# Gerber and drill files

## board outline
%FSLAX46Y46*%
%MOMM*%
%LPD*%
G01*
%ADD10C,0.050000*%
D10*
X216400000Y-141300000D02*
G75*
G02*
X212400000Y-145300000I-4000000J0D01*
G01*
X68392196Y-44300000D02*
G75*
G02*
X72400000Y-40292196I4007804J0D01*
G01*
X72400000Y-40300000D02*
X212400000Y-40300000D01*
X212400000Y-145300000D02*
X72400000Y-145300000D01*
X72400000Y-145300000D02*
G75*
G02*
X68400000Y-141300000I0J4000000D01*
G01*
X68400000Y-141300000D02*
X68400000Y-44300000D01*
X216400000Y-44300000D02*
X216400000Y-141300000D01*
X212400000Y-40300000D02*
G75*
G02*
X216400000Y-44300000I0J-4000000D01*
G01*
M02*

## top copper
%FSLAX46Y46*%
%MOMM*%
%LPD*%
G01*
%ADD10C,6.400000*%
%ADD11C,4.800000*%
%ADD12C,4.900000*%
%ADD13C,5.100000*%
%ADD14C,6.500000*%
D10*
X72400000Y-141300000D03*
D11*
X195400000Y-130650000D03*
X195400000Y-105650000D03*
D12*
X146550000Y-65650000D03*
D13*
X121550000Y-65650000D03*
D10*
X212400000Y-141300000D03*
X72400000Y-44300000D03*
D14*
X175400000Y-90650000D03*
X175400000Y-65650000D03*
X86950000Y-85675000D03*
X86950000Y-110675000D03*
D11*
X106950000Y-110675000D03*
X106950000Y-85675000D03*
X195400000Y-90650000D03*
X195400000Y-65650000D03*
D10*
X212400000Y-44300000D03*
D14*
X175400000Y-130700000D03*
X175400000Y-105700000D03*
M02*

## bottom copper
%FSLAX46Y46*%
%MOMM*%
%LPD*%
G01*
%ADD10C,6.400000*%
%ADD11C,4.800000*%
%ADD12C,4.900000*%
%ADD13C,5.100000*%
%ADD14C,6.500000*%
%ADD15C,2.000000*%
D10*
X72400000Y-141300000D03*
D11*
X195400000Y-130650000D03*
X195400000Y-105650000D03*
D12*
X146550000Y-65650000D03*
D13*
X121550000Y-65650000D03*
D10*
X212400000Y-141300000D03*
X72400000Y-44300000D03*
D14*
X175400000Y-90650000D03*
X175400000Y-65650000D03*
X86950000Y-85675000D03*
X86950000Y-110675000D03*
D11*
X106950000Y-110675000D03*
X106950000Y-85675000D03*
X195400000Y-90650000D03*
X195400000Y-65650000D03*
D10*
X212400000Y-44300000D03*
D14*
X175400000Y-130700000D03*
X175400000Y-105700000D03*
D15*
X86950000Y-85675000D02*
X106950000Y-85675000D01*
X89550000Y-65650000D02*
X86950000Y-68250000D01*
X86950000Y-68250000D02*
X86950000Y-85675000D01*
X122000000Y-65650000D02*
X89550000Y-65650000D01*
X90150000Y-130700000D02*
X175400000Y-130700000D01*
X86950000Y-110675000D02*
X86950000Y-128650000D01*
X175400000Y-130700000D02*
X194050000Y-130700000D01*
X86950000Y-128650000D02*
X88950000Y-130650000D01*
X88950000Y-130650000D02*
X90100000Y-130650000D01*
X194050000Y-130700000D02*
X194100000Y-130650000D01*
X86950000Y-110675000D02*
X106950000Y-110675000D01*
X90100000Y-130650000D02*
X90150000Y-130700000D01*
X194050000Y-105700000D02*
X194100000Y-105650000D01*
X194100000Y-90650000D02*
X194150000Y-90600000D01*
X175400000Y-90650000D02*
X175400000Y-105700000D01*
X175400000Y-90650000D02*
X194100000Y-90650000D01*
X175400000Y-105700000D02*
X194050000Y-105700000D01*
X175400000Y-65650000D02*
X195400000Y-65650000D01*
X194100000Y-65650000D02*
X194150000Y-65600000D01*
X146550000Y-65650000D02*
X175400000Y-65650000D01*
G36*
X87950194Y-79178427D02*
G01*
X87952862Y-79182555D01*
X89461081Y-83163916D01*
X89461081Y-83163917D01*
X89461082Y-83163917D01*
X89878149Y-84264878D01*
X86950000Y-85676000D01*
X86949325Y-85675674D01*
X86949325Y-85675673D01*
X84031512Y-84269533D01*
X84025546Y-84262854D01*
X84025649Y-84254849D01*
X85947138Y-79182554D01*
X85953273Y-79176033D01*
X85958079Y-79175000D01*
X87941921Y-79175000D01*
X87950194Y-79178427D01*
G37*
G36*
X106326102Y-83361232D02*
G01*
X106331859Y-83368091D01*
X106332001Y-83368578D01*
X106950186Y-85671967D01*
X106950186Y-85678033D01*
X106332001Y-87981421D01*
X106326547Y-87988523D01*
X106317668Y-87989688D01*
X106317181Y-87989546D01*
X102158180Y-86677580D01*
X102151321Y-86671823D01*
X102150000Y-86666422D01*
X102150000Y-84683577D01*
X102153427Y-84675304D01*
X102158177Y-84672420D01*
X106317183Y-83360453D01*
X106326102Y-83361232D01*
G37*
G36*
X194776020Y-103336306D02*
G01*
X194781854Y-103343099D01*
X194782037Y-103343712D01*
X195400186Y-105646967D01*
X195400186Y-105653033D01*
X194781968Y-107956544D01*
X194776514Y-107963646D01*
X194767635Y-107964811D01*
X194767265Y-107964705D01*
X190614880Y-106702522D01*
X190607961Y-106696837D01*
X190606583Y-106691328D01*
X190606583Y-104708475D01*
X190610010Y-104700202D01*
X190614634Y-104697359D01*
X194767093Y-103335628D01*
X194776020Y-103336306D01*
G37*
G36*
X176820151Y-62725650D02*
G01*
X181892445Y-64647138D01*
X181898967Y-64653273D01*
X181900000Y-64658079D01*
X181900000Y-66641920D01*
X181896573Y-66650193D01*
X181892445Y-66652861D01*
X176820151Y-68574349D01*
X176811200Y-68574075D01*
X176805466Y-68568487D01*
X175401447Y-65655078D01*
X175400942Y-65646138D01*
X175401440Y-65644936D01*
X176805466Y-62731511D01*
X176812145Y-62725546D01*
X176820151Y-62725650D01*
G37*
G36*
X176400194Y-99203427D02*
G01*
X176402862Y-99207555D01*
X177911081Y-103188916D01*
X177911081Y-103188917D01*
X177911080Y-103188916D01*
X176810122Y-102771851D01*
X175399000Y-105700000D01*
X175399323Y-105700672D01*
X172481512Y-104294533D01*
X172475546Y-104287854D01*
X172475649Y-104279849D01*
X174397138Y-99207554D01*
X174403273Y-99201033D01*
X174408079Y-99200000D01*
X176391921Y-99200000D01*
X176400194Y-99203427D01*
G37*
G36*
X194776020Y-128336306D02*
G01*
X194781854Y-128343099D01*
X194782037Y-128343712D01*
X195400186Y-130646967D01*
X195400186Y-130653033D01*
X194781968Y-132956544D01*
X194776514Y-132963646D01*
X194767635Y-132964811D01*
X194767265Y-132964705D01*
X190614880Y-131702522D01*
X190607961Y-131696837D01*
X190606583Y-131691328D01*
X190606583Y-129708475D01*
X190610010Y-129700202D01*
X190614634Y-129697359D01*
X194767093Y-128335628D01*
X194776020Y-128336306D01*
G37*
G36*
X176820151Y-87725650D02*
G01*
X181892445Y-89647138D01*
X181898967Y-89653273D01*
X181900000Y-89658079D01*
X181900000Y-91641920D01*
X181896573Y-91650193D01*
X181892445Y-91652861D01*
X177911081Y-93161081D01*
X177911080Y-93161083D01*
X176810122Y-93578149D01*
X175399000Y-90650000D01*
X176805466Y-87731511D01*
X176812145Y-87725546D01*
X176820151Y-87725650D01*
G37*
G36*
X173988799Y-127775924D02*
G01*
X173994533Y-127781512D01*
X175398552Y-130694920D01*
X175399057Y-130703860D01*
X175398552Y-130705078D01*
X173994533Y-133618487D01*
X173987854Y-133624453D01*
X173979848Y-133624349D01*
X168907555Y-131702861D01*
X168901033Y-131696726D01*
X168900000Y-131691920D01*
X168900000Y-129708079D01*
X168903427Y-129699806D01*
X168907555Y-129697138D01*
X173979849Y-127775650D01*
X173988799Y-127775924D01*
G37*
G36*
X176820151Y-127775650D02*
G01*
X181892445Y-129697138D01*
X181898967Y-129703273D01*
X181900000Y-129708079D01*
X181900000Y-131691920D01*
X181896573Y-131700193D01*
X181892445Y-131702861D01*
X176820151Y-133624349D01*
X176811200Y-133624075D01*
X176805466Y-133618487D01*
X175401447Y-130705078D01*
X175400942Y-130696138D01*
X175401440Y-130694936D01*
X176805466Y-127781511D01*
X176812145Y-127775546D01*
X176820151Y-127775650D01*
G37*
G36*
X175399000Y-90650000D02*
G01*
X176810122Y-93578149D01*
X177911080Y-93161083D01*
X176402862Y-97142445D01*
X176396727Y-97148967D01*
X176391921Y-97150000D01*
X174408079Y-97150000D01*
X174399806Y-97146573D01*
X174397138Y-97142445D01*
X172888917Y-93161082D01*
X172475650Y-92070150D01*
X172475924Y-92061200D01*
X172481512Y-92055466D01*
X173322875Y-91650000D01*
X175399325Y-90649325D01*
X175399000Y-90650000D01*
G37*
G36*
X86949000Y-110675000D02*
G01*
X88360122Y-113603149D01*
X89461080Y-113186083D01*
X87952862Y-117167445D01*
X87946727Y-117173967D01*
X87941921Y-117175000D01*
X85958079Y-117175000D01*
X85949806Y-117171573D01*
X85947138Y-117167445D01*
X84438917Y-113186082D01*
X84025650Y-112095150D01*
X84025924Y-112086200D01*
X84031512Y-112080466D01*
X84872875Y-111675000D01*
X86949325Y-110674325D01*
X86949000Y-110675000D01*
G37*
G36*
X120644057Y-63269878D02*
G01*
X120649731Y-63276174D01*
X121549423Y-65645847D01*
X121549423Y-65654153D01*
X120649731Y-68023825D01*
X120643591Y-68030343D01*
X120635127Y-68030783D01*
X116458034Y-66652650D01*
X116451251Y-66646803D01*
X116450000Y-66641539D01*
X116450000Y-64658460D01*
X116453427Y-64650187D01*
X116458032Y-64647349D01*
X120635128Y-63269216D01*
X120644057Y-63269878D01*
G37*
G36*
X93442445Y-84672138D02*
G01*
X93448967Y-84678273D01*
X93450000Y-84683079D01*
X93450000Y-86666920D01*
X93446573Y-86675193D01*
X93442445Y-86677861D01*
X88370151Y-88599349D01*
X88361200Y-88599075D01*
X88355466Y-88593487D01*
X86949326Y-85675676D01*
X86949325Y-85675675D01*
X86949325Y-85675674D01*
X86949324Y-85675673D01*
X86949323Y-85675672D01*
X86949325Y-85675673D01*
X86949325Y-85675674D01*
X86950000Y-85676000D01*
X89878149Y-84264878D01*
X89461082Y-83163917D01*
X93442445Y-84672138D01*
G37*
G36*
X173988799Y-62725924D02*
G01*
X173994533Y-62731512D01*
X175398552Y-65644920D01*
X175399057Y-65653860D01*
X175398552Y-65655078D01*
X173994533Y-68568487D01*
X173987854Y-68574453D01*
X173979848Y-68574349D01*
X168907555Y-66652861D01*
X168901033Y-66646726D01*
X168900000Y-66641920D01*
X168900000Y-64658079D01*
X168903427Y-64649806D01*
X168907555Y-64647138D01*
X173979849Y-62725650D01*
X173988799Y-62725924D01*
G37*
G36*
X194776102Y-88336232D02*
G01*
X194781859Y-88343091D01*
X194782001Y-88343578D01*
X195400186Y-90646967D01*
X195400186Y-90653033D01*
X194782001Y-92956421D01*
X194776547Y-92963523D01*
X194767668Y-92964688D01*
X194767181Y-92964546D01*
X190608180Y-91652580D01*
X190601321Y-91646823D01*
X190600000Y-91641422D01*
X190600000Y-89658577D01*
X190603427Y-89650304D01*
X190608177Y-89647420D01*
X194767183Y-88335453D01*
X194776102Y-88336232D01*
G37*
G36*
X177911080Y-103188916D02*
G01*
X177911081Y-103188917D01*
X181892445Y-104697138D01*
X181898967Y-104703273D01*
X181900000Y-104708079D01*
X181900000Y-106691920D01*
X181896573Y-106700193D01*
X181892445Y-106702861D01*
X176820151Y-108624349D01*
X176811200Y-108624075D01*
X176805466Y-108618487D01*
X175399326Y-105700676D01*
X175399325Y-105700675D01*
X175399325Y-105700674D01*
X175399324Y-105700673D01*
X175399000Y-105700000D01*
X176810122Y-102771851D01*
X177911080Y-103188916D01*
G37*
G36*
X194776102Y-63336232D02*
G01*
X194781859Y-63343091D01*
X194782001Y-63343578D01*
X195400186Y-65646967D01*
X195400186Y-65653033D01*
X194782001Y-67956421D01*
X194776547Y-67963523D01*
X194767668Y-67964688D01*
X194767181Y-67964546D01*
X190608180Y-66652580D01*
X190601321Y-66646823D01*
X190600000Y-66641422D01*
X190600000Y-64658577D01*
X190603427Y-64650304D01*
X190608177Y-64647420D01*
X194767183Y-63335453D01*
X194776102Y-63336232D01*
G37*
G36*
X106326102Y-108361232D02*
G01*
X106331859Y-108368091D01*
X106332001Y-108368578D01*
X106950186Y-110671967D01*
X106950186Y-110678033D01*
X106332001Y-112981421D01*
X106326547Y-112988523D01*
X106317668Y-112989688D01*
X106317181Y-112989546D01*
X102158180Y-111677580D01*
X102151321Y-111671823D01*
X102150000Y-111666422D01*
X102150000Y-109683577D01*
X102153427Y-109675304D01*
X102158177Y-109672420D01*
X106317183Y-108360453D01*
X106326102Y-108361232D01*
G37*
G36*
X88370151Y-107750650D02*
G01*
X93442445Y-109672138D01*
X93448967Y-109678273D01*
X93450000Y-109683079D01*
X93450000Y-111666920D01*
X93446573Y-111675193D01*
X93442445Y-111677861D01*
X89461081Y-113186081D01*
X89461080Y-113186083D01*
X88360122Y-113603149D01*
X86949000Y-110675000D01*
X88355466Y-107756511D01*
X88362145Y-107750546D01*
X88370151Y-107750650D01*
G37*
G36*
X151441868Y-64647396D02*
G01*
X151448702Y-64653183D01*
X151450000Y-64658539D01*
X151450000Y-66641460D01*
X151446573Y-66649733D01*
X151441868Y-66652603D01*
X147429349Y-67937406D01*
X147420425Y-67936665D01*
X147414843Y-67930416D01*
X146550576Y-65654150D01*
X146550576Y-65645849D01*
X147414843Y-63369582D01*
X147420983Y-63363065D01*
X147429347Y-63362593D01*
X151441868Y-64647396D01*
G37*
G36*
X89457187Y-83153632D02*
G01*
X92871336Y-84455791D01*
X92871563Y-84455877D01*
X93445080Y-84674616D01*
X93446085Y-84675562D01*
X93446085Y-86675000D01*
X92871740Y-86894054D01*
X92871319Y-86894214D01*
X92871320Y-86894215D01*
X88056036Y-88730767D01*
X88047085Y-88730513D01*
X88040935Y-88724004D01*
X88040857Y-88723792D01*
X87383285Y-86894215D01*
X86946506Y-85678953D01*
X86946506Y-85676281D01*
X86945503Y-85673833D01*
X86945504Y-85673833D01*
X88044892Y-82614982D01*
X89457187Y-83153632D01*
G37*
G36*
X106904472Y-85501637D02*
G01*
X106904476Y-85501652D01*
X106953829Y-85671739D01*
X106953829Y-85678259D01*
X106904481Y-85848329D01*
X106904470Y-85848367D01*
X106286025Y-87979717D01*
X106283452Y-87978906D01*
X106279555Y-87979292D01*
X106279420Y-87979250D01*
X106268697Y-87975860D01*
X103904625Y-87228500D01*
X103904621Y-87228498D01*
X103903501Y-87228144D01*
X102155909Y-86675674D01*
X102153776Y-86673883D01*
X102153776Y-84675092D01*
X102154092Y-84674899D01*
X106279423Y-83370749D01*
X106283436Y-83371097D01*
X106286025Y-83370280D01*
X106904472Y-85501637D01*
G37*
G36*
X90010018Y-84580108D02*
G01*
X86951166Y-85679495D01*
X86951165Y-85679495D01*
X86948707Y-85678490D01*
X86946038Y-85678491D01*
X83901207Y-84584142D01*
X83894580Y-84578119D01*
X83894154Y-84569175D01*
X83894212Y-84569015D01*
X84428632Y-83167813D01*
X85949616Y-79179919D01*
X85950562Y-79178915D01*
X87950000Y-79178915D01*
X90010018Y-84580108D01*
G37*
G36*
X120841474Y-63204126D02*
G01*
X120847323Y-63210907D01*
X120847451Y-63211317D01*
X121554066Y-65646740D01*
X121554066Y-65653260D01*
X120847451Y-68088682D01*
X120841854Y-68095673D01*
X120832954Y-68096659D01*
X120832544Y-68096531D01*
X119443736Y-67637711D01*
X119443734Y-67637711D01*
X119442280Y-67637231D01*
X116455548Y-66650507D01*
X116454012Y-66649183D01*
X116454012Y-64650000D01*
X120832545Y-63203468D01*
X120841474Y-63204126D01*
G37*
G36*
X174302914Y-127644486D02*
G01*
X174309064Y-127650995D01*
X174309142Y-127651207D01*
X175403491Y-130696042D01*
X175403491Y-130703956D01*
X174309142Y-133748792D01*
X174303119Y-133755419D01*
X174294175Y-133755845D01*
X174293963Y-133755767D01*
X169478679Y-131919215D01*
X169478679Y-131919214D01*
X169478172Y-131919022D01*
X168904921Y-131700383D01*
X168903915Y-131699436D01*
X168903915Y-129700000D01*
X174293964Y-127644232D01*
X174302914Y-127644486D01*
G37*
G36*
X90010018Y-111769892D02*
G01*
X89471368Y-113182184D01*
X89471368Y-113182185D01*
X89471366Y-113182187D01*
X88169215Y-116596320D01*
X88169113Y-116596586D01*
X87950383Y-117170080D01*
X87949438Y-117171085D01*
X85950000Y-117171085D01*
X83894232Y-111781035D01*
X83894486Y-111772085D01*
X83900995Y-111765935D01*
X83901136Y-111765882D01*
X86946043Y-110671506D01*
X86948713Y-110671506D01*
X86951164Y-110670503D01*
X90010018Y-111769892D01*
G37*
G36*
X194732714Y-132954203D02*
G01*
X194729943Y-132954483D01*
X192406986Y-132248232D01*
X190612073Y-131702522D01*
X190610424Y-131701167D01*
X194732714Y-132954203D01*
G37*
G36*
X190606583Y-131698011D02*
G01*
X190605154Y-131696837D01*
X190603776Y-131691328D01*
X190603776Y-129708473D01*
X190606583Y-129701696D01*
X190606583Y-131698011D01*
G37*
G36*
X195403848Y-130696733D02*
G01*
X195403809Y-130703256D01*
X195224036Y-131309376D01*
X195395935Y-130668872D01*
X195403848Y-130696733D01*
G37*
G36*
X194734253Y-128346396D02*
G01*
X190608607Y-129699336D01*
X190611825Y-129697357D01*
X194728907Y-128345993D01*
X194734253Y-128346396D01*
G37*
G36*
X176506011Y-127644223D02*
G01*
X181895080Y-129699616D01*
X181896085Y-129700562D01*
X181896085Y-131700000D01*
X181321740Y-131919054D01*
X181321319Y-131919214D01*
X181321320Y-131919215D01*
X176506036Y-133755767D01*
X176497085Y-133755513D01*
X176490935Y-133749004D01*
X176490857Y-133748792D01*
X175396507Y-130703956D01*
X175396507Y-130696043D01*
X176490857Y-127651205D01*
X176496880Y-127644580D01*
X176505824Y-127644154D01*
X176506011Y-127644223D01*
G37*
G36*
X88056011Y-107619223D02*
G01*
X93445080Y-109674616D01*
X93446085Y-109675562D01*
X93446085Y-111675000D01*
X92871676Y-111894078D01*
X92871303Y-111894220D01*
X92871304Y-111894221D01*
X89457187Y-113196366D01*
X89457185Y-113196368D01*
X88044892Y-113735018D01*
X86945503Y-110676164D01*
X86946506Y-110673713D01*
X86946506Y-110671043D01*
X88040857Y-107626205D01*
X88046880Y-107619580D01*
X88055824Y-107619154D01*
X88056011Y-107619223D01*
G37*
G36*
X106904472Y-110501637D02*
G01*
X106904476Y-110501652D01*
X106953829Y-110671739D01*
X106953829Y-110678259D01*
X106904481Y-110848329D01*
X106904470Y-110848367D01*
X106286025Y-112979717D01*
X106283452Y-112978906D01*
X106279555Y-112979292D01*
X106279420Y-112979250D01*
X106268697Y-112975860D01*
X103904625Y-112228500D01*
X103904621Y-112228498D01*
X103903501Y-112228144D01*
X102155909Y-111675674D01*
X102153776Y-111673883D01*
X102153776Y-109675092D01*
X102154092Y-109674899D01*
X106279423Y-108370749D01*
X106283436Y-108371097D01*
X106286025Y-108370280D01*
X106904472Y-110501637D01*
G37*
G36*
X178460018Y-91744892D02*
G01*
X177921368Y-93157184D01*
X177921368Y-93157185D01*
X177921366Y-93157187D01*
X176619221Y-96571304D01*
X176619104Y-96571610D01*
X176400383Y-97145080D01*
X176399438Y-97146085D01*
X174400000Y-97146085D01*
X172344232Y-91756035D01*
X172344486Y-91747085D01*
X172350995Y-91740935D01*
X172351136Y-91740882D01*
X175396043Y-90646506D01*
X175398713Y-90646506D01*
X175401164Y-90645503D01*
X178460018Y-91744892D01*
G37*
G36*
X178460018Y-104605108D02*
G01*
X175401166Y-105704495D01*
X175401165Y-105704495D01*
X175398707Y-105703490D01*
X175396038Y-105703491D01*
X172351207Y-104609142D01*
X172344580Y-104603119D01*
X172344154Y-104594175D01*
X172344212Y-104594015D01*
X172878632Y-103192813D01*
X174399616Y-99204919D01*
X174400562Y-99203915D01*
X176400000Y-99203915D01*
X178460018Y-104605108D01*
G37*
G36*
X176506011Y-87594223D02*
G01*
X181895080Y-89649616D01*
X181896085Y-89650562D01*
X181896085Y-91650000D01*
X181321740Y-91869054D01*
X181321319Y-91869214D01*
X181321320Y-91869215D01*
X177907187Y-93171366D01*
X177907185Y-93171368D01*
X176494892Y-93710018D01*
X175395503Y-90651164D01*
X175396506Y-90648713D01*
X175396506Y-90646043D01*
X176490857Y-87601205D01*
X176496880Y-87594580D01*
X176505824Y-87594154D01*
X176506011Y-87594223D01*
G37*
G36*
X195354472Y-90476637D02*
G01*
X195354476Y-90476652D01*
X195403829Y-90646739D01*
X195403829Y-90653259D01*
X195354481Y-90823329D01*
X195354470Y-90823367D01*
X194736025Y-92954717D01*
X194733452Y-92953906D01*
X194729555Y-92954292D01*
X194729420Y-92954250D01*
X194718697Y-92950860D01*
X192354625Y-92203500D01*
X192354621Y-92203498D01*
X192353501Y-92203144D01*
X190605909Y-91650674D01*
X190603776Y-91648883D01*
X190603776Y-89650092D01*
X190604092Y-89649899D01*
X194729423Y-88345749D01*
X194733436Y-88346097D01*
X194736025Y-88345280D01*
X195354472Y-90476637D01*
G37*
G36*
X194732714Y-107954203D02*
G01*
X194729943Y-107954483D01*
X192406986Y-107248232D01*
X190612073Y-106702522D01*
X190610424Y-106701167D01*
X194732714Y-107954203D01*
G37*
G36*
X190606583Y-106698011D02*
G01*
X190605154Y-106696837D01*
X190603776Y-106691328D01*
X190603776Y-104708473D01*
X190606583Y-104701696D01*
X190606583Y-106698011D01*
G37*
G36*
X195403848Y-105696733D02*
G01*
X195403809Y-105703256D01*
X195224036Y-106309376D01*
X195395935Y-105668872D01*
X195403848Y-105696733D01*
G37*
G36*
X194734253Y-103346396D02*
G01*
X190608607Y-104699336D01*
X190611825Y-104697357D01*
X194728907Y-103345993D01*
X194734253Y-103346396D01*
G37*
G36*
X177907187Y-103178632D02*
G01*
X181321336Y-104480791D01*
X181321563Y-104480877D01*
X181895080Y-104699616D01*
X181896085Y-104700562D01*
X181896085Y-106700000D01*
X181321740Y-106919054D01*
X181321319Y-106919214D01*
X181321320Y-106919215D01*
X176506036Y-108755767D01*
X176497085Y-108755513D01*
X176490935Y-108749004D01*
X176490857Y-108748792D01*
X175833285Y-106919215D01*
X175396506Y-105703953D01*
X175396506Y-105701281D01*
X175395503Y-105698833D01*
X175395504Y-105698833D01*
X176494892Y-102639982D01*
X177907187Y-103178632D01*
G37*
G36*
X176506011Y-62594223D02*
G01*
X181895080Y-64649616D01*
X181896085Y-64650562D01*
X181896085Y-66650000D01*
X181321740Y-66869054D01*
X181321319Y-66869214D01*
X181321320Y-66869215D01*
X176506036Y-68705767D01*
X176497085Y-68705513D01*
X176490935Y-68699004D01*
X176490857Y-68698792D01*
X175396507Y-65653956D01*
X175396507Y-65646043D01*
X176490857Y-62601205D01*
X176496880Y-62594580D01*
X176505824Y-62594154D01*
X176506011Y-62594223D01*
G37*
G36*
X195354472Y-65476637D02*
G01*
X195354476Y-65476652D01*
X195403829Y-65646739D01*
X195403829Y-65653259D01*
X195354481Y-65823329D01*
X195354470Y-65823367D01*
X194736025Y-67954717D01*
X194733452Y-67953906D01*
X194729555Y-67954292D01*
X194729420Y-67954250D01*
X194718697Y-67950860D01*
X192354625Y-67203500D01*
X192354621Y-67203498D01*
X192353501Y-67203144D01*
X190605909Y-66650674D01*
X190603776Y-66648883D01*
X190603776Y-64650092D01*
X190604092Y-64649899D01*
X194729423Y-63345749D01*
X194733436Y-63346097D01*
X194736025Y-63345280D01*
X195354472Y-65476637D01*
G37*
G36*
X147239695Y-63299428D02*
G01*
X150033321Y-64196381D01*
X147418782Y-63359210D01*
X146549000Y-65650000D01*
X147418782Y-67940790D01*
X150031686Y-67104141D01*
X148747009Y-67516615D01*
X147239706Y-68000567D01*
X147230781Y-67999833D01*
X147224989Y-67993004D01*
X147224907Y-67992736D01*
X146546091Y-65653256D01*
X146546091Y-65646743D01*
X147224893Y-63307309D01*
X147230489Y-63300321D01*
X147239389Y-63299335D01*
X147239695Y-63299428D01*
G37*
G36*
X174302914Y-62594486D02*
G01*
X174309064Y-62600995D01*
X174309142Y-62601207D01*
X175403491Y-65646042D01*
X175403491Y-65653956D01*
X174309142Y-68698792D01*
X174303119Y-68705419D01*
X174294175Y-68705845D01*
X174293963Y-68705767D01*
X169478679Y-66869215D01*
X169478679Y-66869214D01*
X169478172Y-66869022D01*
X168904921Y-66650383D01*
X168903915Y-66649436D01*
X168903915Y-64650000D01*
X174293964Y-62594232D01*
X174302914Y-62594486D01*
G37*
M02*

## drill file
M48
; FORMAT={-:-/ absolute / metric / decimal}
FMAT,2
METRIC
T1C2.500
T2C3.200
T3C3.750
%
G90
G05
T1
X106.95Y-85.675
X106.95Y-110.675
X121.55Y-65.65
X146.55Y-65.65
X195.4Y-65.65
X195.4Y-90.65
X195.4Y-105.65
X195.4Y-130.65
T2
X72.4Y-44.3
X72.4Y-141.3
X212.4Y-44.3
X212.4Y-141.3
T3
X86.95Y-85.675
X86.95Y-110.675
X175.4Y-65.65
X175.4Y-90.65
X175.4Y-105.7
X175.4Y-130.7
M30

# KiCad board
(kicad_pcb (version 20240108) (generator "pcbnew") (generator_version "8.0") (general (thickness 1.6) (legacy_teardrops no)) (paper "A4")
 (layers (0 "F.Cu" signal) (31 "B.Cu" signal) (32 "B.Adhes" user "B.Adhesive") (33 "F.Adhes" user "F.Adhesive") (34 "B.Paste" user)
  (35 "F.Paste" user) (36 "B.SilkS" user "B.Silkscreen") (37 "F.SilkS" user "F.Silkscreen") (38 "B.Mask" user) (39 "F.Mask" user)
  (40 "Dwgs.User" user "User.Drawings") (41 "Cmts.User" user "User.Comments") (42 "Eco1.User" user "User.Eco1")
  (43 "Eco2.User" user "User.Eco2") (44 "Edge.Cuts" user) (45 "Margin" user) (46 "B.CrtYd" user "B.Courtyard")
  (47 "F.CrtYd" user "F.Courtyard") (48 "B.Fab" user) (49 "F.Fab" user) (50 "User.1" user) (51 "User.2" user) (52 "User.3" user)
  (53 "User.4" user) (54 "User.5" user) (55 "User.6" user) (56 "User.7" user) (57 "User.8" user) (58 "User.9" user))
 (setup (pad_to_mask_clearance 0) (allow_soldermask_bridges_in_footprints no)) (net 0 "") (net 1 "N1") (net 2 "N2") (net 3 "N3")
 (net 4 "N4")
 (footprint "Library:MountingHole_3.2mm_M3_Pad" (layer "F.Cu") (at 72.4 141.3)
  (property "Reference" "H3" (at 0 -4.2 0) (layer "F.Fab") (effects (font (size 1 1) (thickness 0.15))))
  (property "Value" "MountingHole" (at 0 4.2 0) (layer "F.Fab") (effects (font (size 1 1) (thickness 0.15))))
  (pad "1" thru_hole circle (at 0 0) (size 6.4 6.4) (drill 3.2) (layers "*.Cu" "*.Mask") (remove_unused_layers no)))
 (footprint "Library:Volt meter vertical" (layer "F.Cu") (at 195.4 118.15)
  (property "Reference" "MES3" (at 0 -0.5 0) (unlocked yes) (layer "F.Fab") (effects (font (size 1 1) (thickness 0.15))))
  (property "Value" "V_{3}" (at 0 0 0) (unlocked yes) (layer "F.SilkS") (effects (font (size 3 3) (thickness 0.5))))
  (pad "1" thru_hole circle (at 0 12.5 180) (size 4.8 4.8) (drill 2.5) (layers "*.Cu" "*.Mask") (remove_unused_layers no) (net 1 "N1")
   (teardrops (best_length_ratio 0.5) (max_length 8) (best_width_ratio 1) (max_width 8) (curve_points 0) (filter_ratio 0.9) (enabled yes)
    (allow_two_segments yes) (prefer_zone_connections yes)))
  (pad "2" thru_hole circle (at 0 -12.5 180) (size 4.8 4.8) (drill 2.5) (layers "*.Cu" "*.Mask") (remove_unused_layers no) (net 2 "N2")
   (teardrops (best_length_ratio 0.5) (max_length 8) (best_width_ratio 1) (max_width 8) (curve_points 0) (filter_ratio 0.9) (enabled yes)
    (allow_two_segments yes) (prefer_zone_connections yes))))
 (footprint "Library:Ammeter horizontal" (layer "F.Cu") (at 134.05 65.65)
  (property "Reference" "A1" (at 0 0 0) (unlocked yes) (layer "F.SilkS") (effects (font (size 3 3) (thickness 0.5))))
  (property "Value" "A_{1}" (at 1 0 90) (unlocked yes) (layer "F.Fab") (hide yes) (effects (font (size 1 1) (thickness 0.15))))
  (pad "1" thru_hole circle (at 12.5 0 270) (size 4.9 4.9) (drill 2.5) (layers "*.Cu" "*.Mask") (remove_unused_layers no) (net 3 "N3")
   (teardrops (best_length_ratio 0.5) (max_length 8) (best_width_ratio 1) (max_width 8) (curve_points 0) (filter_ratio 0.9) (enabled yes)
    (allow_two_segments yes) (prefer_zone_connections yes)))
  (pad "2" thru_hole circle (at -12.5 0 270) (size 5.1 5.1) (drill 2.5) (layers "*.Cu" "*.Mask") (remove_unused_layers no) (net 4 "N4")
   (teardrops (best_length_ratio 0.5) (max_length 8) (best_width_ratio 1) (max_width 8) (curve_points 0) (filter_ratio 0.9) (enabled yes)
    (allow_two_segments yes) (prefer_zone_connections yes))))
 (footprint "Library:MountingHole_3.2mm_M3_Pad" (layer "F.Cu") (at 212.4 141.3)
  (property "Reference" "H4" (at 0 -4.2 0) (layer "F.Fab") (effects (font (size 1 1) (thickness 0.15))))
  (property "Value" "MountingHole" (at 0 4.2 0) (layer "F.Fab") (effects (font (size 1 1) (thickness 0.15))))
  (pad "1" thru_hole circle (at 0 0) (size 6.4 6.4) (drill 3.2) (layers "*.Cu" "*.Mask") (remove_unused_layers no)))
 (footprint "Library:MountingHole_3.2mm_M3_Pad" (layer "F.Cu") (at 72.4 44.3)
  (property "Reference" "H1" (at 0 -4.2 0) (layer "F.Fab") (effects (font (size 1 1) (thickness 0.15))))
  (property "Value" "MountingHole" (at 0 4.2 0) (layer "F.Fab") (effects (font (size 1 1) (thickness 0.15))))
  (pad "1" thru_hole circle (at 0 0) (size 6.4 6.4) (drill 3.2) (layers "*.Cu" "*.Mask") (remove_unused_layers no)))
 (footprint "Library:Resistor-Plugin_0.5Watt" (layer "F.Cu") (at 175.4 78.15 180)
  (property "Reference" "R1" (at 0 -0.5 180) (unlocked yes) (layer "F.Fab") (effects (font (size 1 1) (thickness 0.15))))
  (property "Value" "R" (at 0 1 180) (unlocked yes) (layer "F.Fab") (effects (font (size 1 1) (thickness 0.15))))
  (pad "1" thru_hole circle (at 0 -12.5 180) (size 6.5 6.5) (drill 3.75) (layers "*.Cu" "*.Mask") (remove_unused_layers no) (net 2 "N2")
   (teardrops (best_length_ratio 0.5) (max_length 8) (best_width_ratio 1) (max_width 8) (curve_points 0) (filter_ratio 0.9) (enabled yes)
    (allow_two_segments yes) (prefer_zone_connections yes)))
  (pad "2" thru_hole circle (at 0 12.5 180) (size 6.5 6.5) (drill 3.75) (layers "*.Cu" "*.Mask") (remove_unused_layers no) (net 3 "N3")
   (teardrops (best_length_ratio 0.5) (max_length 8) (best_width_ratio 1) (max_width 8) (curve_points 0) (filter_ratio 0.9) (enabled yes)
    (allow_two_segments yes) (prefer_zone_connections yes))))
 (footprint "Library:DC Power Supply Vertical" (layer "F.Cu") (at 86.95 98.175)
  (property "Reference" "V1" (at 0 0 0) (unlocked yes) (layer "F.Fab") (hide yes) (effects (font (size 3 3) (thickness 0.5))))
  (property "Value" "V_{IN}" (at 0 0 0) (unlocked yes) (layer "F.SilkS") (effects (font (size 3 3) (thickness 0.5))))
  (pad "1" thru_hole circle (at 0 -12.5) (size 6.5 6.5) (drill 3.75) (layers "*.Cu" "*.Mask") (remove_unused_layers no) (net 4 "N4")
   (teardrops (best_length_ratio 0.5) (max_length 8) (best_width_ratio 1) (max_width 8) (curve_points 0) (filter_ratio 0.9) (enabled yes)
    (allow_two_segments yes) (prefer_zone_connections yes)))
  (pad "2" thru_hole circle (at 0 12.5) (size 6.5 6.5) (drill 3.75) (layers "*.Cu" "*.Mask") (remove_unused_layers no) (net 1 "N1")
   (teardrops (best_length_ratio 0.5) (max_length 8) (best_width_ratio 1) (max_width 8) (curve_points 0) (filter_ratio 0.9) (enabled yes)
    (allow_two_segments yes) (prefer_zone_connections yes))))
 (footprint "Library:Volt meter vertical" (layer "F.Cu") (at 106.95 98.175)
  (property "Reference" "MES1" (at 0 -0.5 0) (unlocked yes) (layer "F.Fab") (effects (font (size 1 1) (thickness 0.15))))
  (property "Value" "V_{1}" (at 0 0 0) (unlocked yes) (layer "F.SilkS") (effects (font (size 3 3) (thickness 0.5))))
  (pad "1" thru_hole circle (at 0 12.5 180) (size 4.8 4.8) (drill 2.5) (layers "*.Cu" "*.Mask") (remove_unused_layers no) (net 1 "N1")
   (teardrops (best_length_ratio 0.5) (max_length 8) (best_width_ratio 1) (max_width 8) (curve_points 0) (filter_ratio 0.9) (enabled yes)
    (allow_two_segments yes) (prefer_zone_connections yes)))
  (pad "2" thru_hole circle (at 0 -12.5 180) (size 4.8 4.8) (drill 2.5) (layers "*.Cu" "*.Mask") (remove_unused_layers no) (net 4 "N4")
   (teardrops (best_length_ratio 0.5) (max_length 8) (best_width_ratio 1) (max_width 8) (curve_points 0) (filter_ratio 0.9) (enabled yes)
    (allow_two_segments yes) (prefer_zone_connections yes))))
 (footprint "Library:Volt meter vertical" (layer "F.Cu") (at 195.4 78.15)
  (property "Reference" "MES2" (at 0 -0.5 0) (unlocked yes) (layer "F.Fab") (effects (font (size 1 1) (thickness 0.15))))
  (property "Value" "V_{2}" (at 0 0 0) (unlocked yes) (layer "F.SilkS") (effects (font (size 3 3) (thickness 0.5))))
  (pad "1" thru_hole circle (at 0 12.5 180) (size 4.8 4.8) (drill 2.5) (layers "*.Cu" "*.Mask") (remove_unused_layers no) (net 2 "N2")
   (teardrops (best_length_ratio 0.5) (max_length 8) (best_width_ratio 1) (max_width 8) (curve_points 0) (filter_ratio 0.9) (enabled yes)
    (allow_two_segments yes) (prefer_zone_connections yes)))
  (pad "2" thru_hole circle (at 0 -12.5 180) (size 4.8 4.8) (drill 2.5) (layers "*.Cu" "*.Mask") (remove_unused_layers no) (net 3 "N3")
   (teardrops (best_length_ratio 0.5) (max_length 8) (best_width_ratio 1) (max_width 8) (curve_points 0) (filter_ratio 0.9) (enabled yes)
    (allow_two_segments yes) (prefer_zone_connections yes))))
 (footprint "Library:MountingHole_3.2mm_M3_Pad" (layer "F.Cu") (at 212.4 44.3)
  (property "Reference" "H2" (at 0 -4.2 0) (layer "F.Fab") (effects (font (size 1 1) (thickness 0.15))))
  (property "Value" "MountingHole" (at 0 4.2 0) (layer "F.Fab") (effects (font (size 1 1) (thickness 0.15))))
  (pad "1" thru_hole circle (at 0 0) (size 6.4 6.4) (drill 3.2) (layers "*.Cu" "*.Mask") (remove_unused_layers no)))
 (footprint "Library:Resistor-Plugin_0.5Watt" (layer "F.Cu") (at 175.4 118.2 180)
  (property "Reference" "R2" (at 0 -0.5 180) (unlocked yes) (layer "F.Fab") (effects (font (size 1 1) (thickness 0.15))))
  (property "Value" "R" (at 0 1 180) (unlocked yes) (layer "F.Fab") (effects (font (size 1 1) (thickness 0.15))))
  (pad "1" thru_hole circle (at 0 -12.5 180) (size 6.5 6.5) (drill 3.75) (layers "*.Cu" "*.Mask") (remove_unused_layers no) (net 1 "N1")
   (teardrops (best_length_ratio 0.5) (max_length 8) (best_width_ratio 1) (max_width 8) (curve_points 0) (filter_ratio 0.9) (enabled yes)
    (allow_two_segments yes) (prefer_zone_connections yes)))
  (pad "2" thru_hole circle (at 0 12.5 180) (size 6.5 6.5) (drill 3.75) (layers "*.Cu" "*.Mask") (remove_unused_layers no) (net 2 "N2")
   (teardrops (best_length_ratio 0.5) (max_length 8) (best_width_ratio 1) (max_width 8) (curve_points 0) (filter_ratio 0.9) (enabled yes)
    (allow_two_segments yes) (prefer_zone_connections yes))))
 (gr_arc (start 216.4 141.3) (mid 215.228427 144.128427) (end 212.4 145.3) (stroke (width 0.05) (type default)) (layer "Edge.Cuts"))
 (gr_arc (start 68.392196 44.3) (mid 69.566055 41.466055) (end 72.4 40.292196) (stroke (width 0.05) (type default)) (layer "Edge.Cuts"))
 (gr_line (start 72.4 40.3) (end 212.4 40.3) (stroke (width 0.05) (type default)) (layer "Edge.Cuts"))
 (gr_line (start 212.4 145.3) (end 72.4 145.3) (stroke (width 0.05) (type default)) (layer "Edge.Cuts"))
 (gr_arc (start 72.4 145.3) (mid 69.571573 144.128427) (end 68.4 141.3) (stroke (width 0.05) (type default)) (layer "Edge.Cuts"))
 (gr_line (start 68.4 141.3) (end 68.4 44.3) (stroke (width 0.05) (type default)) (layer "Edge.Cuts"))
 (gr_line (start 216.4 44.3) (end 216.4 141.3) (stroke (width 0.05) (type default)) (layer "Edge.Cuts"))
 (gr_arc (start 212.4 40.3) (mid 215.228427 41.471573) (end 216.4 44.3) (stroke (width 0.05) (type default)) (layer "Edge.Cuts"))
 (segment (start 86.95 85.675) (end 106.95 85.675) (width 2) (layer "B.Cu") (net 4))
 (segment (start 89.55 65.65) (end 86.95 68.25) (width 2) (layer "B.Cu") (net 4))
 (segment (start 86.95 68.25) (end 86.95 85.675) (width 2) (layer "B.Cu") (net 4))
 (segment (start 122 65.65) (end 89.55 65.65) (width 2) (layer "B.Cu") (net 4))
 (segment (start 90.15 130.7) (end 175.4 130.7) (width 2) (layer "B.Cu") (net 1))
 (segment (start 86.95 110.675) (end 86.95 128.65) (width 2) (layer "B.Cu") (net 1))
 (segment (start 175.4 130.7) (end 194.05 130.7) (width 2) (layer "B.Cu") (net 1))
 (segment (start 86.95 128.65) (end 88.95 130.65) (width 2) (layer "B.Cu") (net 1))
 (segment (start 88.95 130.65) (end 90.1 130.65) (width 2) (layer "B.Cu") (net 1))
 (segment (start 194.05 130.7) (end 194.1 130.65) (width 2) (layer "B.Cu") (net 1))
 (segment (start 86.95 110.675) (end 106.95 110.675) (width 2) (layer "B.Cu") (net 1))
 (segment (start 90.1 130.65) (end 90.15 130.7) (width 2) (layer "B.Cu") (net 1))
 (segment (start 194.05 105.7) (end 194.1 105.65) (width 2) (layer "B.Cu") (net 2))
 (segment (start 194.1 90.65) (end 194.15 90.6) (width 2) (layer "B.Cu") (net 2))
 (segment (start 175.4 90.65) (end 175.4 105.7) (width 2) (layer "B.Cu") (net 2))
 (segment (start 175.4 90.65) (end 194.1 90.65) (width 2) (layer "B.Cu") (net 2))
 (segment (start 175.4 105.7) (end 194.05 105.7) (width 2) (layer "B.Cu") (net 2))
 (segment (start 175.4 65.65) (end 195.4 65.65) (width 2) (layer "B.Cu") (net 3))
 (segment (start 194.1 65.65) (end 194.15 65.6) (width 2) (layer "B.Cu") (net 3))
 (segment (start 146.55 65.65) (end 175.4 65.65) (width 2) (layer "B.Cu") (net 3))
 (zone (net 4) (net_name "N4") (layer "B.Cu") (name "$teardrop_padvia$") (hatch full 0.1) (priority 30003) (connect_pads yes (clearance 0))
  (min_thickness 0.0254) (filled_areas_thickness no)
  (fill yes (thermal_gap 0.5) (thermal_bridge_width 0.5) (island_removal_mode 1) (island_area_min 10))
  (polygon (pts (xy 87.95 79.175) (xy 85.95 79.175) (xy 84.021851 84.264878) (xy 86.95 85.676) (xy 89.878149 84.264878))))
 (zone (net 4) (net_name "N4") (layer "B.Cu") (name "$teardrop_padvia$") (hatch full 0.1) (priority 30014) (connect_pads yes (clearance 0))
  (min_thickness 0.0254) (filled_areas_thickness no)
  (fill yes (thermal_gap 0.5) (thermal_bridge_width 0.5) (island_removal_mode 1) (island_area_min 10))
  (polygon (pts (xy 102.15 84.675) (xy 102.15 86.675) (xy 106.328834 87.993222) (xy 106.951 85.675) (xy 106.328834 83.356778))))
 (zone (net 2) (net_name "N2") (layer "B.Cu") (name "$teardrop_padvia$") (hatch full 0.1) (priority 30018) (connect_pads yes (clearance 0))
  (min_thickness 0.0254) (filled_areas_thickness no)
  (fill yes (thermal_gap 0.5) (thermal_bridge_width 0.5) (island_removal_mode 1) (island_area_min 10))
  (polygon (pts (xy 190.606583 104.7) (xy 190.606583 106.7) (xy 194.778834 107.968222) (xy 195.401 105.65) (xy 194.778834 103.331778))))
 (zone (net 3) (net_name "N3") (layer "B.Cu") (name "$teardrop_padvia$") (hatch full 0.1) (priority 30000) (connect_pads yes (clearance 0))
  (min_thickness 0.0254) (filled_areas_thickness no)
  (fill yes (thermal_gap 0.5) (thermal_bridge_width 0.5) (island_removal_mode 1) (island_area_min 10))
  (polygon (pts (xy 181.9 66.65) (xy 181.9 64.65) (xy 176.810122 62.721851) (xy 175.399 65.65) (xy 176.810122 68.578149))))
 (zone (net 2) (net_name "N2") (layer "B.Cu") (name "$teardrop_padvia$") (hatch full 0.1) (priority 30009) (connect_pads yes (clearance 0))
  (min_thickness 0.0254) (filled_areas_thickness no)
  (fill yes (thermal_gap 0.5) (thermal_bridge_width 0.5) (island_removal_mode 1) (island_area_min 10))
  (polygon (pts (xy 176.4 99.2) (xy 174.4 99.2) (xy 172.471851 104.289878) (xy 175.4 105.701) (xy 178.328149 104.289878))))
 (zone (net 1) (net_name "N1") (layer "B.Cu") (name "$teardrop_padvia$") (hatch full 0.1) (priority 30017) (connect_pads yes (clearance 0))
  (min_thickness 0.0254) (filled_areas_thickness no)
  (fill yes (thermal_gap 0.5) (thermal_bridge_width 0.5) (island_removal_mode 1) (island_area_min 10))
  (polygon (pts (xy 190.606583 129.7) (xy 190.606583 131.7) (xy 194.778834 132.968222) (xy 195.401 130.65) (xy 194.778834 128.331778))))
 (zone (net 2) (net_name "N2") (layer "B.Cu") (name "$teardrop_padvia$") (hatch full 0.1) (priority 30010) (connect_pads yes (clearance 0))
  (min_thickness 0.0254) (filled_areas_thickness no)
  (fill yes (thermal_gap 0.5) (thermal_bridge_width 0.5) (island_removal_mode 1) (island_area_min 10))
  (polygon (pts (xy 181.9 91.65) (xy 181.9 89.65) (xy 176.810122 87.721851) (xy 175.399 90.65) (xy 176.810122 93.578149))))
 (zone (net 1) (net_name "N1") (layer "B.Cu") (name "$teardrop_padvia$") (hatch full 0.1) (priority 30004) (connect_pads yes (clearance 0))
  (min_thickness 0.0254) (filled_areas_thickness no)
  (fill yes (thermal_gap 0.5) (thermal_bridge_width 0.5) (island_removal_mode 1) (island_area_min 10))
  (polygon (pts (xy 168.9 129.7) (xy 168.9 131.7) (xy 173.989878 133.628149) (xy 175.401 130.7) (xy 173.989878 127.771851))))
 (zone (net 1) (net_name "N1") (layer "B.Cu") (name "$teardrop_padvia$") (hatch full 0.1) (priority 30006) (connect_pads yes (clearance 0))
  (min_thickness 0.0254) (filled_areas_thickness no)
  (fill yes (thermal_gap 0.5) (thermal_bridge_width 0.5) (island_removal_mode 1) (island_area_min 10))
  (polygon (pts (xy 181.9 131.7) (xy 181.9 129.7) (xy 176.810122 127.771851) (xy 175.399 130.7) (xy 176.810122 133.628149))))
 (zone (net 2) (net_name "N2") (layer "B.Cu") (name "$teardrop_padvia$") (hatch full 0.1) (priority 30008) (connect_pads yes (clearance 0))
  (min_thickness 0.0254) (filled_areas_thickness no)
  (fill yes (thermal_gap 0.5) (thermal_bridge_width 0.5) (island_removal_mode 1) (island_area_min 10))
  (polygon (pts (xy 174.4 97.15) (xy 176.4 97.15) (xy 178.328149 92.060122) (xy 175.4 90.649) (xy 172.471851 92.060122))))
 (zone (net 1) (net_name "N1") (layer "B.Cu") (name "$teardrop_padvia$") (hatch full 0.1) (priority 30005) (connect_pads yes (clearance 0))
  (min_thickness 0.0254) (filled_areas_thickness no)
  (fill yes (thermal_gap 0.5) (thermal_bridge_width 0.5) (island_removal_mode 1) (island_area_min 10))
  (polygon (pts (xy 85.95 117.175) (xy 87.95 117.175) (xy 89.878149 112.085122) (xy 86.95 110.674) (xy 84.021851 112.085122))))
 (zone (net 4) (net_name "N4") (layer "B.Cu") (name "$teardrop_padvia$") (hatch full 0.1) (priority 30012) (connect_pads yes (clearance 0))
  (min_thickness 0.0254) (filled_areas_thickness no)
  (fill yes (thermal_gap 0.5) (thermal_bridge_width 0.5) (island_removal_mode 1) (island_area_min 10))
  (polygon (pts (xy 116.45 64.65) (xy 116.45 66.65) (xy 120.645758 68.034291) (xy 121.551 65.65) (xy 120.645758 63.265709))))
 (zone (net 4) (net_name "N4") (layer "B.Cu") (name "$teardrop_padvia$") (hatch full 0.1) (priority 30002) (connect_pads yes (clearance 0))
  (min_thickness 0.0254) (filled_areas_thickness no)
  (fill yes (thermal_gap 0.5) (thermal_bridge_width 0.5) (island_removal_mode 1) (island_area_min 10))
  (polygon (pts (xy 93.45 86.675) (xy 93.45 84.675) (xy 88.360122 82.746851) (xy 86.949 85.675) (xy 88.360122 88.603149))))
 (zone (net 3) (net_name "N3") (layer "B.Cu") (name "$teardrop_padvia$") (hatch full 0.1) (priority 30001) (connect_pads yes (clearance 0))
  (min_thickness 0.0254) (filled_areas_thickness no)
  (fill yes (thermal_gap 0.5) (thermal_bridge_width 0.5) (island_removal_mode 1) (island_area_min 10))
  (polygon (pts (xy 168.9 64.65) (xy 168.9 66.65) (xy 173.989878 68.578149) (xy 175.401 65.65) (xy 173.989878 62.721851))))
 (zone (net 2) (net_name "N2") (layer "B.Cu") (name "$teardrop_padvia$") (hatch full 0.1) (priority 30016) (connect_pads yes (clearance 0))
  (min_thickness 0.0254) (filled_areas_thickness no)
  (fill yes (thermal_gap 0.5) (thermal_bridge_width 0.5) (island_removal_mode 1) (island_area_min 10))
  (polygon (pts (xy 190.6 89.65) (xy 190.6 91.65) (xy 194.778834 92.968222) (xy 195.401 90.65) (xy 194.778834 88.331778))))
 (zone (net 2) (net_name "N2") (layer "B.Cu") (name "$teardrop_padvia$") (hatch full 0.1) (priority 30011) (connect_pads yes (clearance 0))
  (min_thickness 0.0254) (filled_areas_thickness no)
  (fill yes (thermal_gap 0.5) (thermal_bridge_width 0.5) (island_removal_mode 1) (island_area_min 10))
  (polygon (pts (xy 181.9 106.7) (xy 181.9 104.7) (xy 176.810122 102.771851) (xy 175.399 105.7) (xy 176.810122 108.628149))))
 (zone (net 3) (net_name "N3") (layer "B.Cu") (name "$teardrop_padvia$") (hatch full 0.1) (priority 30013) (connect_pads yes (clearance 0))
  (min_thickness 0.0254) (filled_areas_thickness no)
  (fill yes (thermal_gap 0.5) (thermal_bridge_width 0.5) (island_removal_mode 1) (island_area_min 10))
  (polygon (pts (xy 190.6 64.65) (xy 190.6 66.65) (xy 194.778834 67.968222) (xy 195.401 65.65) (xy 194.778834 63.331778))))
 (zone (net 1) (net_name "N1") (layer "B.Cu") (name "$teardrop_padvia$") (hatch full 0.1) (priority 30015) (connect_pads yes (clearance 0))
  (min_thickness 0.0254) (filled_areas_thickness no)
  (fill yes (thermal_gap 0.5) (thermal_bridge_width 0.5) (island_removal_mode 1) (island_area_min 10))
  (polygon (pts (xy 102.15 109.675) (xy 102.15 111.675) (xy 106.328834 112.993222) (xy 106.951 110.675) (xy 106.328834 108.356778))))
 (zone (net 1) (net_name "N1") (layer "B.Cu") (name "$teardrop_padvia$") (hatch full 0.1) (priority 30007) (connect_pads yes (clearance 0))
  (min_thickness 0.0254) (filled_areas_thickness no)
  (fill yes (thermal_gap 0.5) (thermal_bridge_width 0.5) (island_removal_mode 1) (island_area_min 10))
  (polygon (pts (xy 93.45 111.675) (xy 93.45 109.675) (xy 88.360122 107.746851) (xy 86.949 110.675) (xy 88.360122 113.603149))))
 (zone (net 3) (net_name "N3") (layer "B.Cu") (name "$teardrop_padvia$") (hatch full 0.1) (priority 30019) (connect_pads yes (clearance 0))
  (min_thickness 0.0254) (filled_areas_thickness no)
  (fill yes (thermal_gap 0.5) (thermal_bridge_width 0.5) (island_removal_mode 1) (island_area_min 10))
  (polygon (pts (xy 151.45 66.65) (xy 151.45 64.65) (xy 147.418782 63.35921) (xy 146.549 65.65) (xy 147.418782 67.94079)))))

